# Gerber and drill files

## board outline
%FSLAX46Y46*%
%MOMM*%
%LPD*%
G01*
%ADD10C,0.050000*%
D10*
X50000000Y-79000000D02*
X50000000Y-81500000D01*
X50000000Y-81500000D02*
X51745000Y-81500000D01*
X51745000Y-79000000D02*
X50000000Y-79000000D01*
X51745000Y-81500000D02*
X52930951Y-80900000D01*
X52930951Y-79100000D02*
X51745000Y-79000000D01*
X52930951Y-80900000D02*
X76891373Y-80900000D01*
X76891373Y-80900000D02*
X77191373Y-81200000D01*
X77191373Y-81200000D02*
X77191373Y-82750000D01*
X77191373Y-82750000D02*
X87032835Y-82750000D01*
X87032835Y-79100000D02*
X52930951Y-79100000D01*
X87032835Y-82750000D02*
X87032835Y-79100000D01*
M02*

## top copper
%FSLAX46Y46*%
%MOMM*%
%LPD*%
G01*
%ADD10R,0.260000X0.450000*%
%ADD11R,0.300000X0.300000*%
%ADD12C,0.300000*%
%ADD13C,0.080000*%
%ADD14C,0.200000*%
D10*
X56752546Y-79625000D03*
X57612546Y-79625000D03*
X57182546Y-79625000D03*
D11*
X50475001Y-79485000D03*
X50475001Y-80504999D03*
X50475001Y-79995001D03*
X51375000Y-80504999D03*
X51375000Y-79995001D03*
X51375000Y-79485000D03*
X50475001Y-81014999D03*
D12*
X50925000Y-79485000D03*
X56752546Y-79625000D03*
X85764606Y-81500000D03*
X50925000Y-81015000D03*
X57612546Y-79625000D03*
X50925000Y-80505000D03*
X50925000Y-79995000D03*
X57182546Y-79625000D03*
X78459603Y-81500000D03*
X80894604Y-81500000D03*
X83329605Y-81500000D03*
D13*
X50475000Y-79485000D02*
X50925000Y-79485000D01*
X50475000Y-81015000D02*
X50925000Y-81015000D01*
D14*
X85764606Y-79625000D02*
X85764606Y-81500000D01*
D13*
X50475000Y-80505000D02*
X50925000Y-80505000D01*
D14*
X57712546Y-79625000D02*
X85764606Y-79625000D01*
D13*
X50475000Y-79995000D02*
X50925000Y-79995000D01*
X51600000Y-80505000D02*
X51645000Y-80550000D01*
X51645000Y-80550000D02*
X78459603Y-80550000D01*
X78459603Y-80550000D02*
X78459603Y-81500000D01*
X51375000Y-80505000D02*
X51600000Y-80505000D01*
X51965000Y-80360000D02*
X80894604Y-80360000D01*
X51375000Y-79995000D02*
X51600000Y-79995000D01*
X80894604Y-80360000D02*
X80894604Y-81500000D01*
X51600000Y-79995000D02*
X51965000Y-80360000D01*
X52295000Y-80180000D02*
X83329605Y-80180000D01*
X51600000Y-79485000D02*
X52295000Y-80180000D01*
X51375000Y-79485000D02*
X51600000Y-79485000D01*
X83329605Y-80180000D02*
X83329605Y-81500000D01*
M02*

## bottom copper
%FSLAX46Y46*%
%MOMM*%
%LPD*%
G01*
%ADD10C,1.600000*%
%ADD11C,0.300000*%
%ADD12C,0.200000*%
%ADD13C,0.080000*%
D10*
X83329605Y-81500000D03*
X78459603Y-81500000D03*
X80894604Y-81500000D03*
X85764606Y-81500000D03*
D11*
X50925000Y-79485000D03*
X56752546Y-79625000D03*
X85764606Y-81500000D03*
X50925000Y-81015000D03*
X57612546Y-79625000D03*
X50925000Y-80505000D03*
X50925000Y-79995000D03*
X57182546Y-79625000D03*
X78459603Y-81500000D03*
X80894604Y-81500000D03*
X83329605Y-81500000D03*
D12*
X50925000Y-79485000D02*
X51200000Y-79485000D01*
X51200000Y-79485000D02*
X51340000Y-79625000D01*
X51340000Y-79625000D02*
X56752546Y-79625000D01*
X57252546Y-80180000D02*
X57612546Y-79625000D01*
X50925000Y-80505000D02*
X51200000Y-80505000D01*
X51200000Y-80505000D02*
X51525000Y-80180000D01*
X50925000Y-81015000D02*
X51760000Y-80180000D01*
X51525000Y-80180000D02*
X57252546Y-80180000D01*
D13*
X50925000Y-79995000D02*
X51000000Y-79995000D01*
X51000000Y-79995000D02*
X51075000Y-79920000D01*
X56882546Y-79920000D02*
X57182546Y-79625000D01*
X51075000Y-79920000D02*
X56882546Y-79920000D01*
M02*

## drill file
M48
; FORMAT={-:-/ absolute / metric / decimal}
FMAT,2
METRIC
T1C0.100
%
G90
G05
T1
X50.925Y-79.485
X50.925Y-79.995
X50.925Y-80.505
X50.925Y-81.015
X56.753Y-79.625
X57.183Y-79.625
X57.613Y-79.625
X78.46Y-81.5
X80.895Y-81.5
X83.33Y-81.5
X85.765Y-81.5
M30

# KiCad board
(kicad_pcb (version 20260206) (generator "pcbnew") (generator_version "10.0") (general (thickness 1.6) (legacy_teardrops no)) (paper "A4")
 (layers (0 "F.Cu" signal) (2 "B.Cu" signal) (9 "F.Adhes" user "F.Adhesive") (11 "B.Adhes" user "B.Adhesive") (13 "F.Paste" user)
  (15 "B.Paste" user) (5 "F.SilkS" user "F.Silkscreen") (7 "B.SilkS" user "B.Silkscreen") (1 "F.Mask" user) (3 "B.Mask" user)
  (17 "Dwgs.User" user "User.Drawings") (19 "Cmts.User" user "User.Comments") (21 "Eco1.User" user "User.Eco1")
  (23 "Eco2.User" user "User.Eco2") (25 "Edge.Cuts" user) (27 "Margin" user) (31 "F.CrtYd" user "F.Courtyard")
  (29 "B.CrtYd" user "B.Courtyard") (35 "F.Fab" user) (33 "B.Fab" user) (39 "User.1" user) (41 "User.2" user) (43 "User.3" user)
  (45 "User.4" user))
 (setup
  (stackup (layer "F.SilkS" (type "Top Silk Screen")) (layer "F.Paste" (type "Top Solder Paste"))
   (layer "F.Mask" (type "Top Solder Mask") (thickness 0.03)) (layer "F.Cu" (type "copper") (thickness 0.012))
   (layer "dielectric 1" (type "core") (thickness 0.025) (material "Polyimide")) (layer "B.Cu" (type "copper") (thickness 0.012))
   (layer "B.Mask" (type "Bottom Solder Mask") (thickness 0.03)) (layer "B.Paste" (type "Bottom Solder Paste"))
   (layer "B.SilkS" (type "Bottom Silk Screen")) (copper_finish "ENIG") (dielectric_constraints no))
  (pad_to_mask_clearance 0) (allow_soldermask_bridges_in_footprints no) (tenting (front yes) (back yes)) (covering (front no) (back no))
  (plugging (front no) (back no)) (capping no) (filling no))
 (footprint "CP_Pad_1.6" (layer "F.Cu") (at 85.764606 81.5)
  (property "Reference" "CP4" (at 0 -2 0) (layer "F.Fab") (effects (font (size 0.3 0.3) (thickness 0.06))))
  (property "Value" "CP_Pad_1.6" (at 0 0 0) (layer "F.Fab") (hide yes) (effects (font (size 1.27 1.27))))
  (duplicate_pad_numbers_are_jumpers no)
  (pad "1" smd circle (at 0 0) (size 1.6 1.6) (layers "B.Cu" "B.Mask") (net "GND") (solder_mask_margin 0.1)))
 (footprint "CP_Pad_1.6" (layer "F.Cu") (at 78.459603 81.5)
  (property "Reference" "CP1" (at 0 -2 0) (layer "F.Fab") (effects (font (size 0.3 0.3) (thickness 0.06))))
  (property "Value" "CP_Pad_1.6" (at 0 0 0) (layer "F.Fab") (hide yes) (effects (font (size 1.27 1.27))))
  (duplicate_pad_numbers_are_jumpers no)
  (pad "1" smd circle (at 0 0) (size 1.6 1.6) (layers "B.Cu" "B.Mask") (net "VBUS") (solder_mask_margin 0.1)))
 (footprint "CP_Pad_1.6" (layer "F.Cu") (at 83.329605 81.5)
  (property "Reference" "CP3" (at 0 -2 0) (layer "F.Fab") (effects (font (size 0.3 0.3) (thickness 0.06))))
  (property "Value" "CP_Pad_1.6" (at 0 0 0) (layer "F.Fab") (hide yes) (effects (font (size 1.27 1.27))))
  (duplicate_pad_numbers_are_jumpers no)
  (pad "1" smd circle (at 0 0) (size 1.6 1.6) (layers "B.Cu" "B.Mask") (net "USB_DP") (solder_mask_margin 0.1)))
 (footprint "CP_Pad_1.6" (layer "F.Cu") (at 80.894604 81.5)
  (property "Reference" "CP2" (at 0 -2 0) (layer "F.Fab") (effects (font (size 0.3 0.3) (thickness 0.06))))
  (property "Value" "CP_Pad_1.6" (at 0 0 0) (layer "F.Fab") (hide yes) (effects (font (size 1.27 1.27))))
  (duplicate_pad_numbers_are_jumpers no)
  (pad "1" smd circle (at 0 0) (size 1.6 1.6) (layers "B.Cu" "B.Mask") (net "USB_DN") (solder_mask_margin 0.1)))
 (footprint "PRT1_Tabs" (layer "F.Cu") (at 57.182546 79.625)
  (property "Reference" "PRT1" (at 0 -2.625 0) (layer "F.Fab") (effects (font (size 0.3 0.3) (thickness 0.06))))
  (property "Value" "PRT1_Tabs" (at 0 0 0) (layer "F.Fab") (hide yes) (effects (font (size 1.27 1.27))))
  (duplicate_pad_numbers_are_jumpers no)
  (pad "1" smd rect (at -0.43 0) (size 0.26 0.45) (layers "F.Cu" "F.Mask") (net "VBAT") (solder_mask_margin 0.05) (thermal_bridge_angle 45))
  (pad "2" smd rect (at 0.43 0) (size 0.26 0.45) (layers "F.Cu" "F.Mask") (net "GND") (solder_mask_margin 0.05) (thermal_bridge_angle 45))
  (pad "3" smd rect (at 0 0) (size 0.26 0.45) (layers "F.Cu" "F.Mask") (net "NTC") (solder_mask_margin 0.05) (thermal_bridge_angle 45)))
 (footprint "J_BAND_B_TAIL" (layer "F.Cu") (at 50.9 80.25)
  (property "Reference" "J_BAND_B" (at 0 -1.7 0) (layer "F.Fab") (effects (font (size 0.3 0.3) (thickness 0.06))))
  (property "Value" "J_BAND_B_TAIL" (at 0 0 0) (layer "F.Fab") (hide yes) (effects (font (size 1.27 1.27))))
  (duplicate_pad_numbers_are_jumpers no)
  (pad "1" smd rect (at -0.424999 -0.765) (size 0.3 0.3) (layers "F.Cu" "F.Mask") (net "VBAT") (solder_mask_margin 0.05)
   (thermal_bridge_angle 45))
  (pad "2" smd rect (at -0.424999 0.254999) (size 0.3 0.3) (layers "F.Cu" "F.Mask") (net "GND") (solder_mask_margin 0.05)
   (thermal_bridge_angle 45))
  (pad "3" smd rect (at -0.424999 -0.254999) (size 0.3 0.3) (layers "F.Cu" "F.Mask") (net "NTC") (solder_mask_margin 0.05)
   (thermal_bridge_angle 45))
  (pad "4" smd rect (at 0.475 0.254999) (size 0.3 0.3) (layers "F.Cu" "F.Mask") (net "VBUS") (solder_mask_margin 0.05)
   (thermal_bridge_angle 45))
  (pad "5" smd rect (at 0.475 -0.254999) (size 0.3 0.3) (layers "F.Cu" "F.Mask") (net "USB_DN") (solder_mask_margin 0.05)
   (thermal_bridge_angle 45))
  (pad "6" smd rect (at 0.475 -0.765) (size 0.3 0.3) (layers "F.Cu" "F.Mask") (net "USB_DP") (solder_mask_margin 0.05)
   (thermal_bridge_angle 45))
  (pad "7" smd rect (at -0.424999 0.764999) (size 0.3 0.3) (layers "F.Cu" "F.Mask") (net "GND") (solder_mask_margin 0.05)
   (thermal_bridge_angle 45)))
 (gr_line (start 50 79) (end 50 81.5) (stroke (width 0.05) (type default)) (layer "Edge.Cuts"))
 (gr_line (start 50 81.5) (end 51.745 81.5) (stroke (width 0.05) (type default)) (layer "Edge.Cuts"))
 (gr_line (start 51.745 79) (end 50 79) (stroke (width 0.05) (type default)) (layer "Edge.Cuts"))
 (gr_line (start 51.745 81.5) (end 52.930951 80.9) (stroke (width 0.05) (type default)) (layer "Edge.Cuts"))
 (gr_line (start 52.930951 79.1) (end 51.745 79) (stroke (width 0.05) (type default)) (layer "Edge.Cuts"))
 (gr_line (start 52.930951 80.9) (end 76.891373 80.9) (stroke (width 0.05) (type default)) (layer "Edge.Cuts"))
 (gr_line (start 76.891373 80.9) (end 77.191373 81.2) (stroke (width 0.05) (type default)) (layer "Edge.Cuts"))
 (gr_line (start 77.191373 81.2) (end 77.191373 82.75) (stroke (width 0.05) (type default)) (layer "Edge.Cuts"))
 (gr_line (start 77.191373 82.75) (end 87.032835 82.75) (stroke (width 0.05) (type default)) (layer "Edge.Cuts"))
 (gr_line (start 87.032835 79.1) (end 52.930951 79.1) (stroke (width 0.05) (type default)) (layer "Edge.Cuts"))
 (gr_line (start 87.032835 82.75) (end 87.032835 79.1) (stroke (width 0.05) (type default)) (layer "Edge.Cuts"))
 (segment (start 50.475 79.485) (end 50.925 79.485) (width 0.08) (layer "F.Cu") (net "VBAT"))
 (via (at 50.925 79.485) (size 0.3) (drill 0.1) (layers "F.Cu" "B.Cu") (tenting (front yes) (back yes)) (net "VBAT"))
 (via (at 56.752546 79.625) (size 0.3) (drill 0.1) (layers "F.Cu" "B.Cu") (tenting (front yes) (back yes)) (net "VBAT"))
 (segment (start 50.925 79.485) (end 51.2 79.485) (width 0.2) (layer "B.Cu") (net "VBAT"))
 (segment (start 51.2 79.485) (end 51.34 79.625) (width 0.2) (layer "B.Cu") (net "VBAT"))
 (segment (start 51.34 79.625) (end 56.752546 79.625) (width 0.2) (layer "B.Cu") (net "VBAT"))
 (segment (start 85.764606 79.625) (end 85.764606 81.5) (width 0.2) (layer "F.Cu") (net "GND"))
 (segment (start 50.475 81.015) (end 50.925 81.015) (width 0.08) (layer "F.Cu") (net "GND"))
 (segment (start 50.475 80.505) (end 50.925 80.505) (width 0.08) (layer "F.Cu") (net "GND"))
 (segment (start 57.712546 79.625) (end 85.764606 79.625) (width 0.2) (layer "F.Cu") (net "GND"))
 (via (at 57.612546 79.625) (size 0.3) (drill 0.1) (layers "F.Cu" "B.Cu") (tenting (front yes) (back yes)) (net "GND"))
 (via (at 50.925 81.015) (size 0.3) (drill 0.1) (layers "F.Cu" "B.Cu") (tenting (front yes) (back yes)) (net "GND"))
 (via (at 50.925 80.505) (size 0.3) (drill 0.1) (layers "F.Cu" "B.Cu") (tenting (front yes) (back yes)) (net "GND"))
 (via (at 85.764606 81.5) (size 0.3) (drill 0.1) (layers "F.Cu" "B.Cu") (tenting (front yes) (back yes)) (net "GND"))
 (segment (start 51.2 80.505) (end 51.525 80.18) (width 0.2) (layer "B.Cu") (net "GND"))
 (segment (start 50.925 81.015) (end 51.76 80.18) (width 0.2) (layer "B.Cu") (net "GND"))
 (segment (start 51.525 80.18) (end 57.252546 80.18) (width 0.2) (layer "B.Cu") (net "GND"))
 (segment (start 50.925 80.505) (end 51.2 80.505) (width 0.2) (layer "B.Cu") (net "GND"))
 (segment (start 57.252546 80.18) (end 57.612546 79.625) (width 0.2) (layer "B.Cu") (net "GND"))
 (segment (start 50.475 79.995) (end 50.925 79.995) (width 0.08) (layer "F.Cu") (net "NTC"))
 (via (at 57.182546 79.625) (size 0.3) (drill 0.1) (layers "F.Cu" "B.Cu") (tenting (front yes) (back yes)) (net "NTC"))
 (via (at 50.925 79.995) (size 0.3) (drill 0.1) (layers "F.Cu" "B.Cu") (tenting (front yes) (back yes)) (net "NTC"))
 (segment (start 51 79.995) (end 51.075 79.92) (width 0.08) (layer "B.Cu") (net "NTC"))
 (segment (start 56.882546 79.92) (end 57.182546 79.625) (width 0.08) (layer "B.Cu") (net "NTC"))
 (segment (start 50.925 79.995) (end 51 79.995) (width 0.08) (layer "B.Cu") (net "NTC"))
 (segment (start 51.075 79.92) (end 56.882546 79.92) (width 0.08) (layer "B.Cu") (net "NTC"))
 (segment (start 51.6 80.505) (end 51.645 80.55) (width 0.08) (layer "F.Cu") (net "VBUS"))
 (segment (start 51.375 80.505) (end 51.6 80.505) (width 0.08) (layer "F.Cu") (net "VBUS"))
 (segment (start 78.459603 80.55) (end 78.459603 81.5) (width 0.08) (layer "F.Cu") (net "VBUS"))
 (segment (start 51.645 80.55) (end 78.459603 80.55) (width 0.08) (layer "F.Cu") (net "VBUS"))
 (via (at 78.459603 81.5) (size 0.3) (drill 0.1) (layers "F.Cu" "B.Cu") (tenting (front yes) (back yes)) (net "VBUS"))
 (segment (start 51.375 79.995) (end 51.6 79.995) (width 0.08) (layer "F.Cu") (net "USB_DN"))
 (segment (start 51.965 80.36) (end 80.894604 80.36) (width 0.08) (layer "F.Cu") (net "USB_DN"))
 (segment (start 80.894604 80.36) (end 80.894604 81.5) (width 0.08) (layer "F.Cu") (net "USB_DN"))
 (segment (start 51.6 79.995) (end 51.965 80.36) (width 0.08) (layer "F.Cu") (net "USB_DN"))
 (via (at 80.894604 81.5) (size 0.3) (drill 0.1) (layers "F.Cu" "B.Cu") (tenting (front yes) (back yes)) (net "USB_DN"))
 (segment (start 51.375 79.485) (end 51.6 79.485) (width 0.08) (layer "F.Cu") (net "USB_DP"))
 (segment (start 51.6 79.485) (end 52.295 80.18) (width 0.08) (layer "F.Cu") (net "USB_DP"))
 (segment (start 83.329605 80.18) (end 83.329605 81.5) (width 0.08) (layer "F.Cu") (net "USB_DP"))
 (segment (start 52.295 80.18) (end 83.329605 80.18) (width 0.08) (layer "F.Cu") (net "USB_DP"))
 (via (at 83.329605 81.5) (size 0.3) (drill 0.1) (layers "F.Cu" "B.Cu") (tenting (front yes) (back yes)) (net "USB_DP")))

